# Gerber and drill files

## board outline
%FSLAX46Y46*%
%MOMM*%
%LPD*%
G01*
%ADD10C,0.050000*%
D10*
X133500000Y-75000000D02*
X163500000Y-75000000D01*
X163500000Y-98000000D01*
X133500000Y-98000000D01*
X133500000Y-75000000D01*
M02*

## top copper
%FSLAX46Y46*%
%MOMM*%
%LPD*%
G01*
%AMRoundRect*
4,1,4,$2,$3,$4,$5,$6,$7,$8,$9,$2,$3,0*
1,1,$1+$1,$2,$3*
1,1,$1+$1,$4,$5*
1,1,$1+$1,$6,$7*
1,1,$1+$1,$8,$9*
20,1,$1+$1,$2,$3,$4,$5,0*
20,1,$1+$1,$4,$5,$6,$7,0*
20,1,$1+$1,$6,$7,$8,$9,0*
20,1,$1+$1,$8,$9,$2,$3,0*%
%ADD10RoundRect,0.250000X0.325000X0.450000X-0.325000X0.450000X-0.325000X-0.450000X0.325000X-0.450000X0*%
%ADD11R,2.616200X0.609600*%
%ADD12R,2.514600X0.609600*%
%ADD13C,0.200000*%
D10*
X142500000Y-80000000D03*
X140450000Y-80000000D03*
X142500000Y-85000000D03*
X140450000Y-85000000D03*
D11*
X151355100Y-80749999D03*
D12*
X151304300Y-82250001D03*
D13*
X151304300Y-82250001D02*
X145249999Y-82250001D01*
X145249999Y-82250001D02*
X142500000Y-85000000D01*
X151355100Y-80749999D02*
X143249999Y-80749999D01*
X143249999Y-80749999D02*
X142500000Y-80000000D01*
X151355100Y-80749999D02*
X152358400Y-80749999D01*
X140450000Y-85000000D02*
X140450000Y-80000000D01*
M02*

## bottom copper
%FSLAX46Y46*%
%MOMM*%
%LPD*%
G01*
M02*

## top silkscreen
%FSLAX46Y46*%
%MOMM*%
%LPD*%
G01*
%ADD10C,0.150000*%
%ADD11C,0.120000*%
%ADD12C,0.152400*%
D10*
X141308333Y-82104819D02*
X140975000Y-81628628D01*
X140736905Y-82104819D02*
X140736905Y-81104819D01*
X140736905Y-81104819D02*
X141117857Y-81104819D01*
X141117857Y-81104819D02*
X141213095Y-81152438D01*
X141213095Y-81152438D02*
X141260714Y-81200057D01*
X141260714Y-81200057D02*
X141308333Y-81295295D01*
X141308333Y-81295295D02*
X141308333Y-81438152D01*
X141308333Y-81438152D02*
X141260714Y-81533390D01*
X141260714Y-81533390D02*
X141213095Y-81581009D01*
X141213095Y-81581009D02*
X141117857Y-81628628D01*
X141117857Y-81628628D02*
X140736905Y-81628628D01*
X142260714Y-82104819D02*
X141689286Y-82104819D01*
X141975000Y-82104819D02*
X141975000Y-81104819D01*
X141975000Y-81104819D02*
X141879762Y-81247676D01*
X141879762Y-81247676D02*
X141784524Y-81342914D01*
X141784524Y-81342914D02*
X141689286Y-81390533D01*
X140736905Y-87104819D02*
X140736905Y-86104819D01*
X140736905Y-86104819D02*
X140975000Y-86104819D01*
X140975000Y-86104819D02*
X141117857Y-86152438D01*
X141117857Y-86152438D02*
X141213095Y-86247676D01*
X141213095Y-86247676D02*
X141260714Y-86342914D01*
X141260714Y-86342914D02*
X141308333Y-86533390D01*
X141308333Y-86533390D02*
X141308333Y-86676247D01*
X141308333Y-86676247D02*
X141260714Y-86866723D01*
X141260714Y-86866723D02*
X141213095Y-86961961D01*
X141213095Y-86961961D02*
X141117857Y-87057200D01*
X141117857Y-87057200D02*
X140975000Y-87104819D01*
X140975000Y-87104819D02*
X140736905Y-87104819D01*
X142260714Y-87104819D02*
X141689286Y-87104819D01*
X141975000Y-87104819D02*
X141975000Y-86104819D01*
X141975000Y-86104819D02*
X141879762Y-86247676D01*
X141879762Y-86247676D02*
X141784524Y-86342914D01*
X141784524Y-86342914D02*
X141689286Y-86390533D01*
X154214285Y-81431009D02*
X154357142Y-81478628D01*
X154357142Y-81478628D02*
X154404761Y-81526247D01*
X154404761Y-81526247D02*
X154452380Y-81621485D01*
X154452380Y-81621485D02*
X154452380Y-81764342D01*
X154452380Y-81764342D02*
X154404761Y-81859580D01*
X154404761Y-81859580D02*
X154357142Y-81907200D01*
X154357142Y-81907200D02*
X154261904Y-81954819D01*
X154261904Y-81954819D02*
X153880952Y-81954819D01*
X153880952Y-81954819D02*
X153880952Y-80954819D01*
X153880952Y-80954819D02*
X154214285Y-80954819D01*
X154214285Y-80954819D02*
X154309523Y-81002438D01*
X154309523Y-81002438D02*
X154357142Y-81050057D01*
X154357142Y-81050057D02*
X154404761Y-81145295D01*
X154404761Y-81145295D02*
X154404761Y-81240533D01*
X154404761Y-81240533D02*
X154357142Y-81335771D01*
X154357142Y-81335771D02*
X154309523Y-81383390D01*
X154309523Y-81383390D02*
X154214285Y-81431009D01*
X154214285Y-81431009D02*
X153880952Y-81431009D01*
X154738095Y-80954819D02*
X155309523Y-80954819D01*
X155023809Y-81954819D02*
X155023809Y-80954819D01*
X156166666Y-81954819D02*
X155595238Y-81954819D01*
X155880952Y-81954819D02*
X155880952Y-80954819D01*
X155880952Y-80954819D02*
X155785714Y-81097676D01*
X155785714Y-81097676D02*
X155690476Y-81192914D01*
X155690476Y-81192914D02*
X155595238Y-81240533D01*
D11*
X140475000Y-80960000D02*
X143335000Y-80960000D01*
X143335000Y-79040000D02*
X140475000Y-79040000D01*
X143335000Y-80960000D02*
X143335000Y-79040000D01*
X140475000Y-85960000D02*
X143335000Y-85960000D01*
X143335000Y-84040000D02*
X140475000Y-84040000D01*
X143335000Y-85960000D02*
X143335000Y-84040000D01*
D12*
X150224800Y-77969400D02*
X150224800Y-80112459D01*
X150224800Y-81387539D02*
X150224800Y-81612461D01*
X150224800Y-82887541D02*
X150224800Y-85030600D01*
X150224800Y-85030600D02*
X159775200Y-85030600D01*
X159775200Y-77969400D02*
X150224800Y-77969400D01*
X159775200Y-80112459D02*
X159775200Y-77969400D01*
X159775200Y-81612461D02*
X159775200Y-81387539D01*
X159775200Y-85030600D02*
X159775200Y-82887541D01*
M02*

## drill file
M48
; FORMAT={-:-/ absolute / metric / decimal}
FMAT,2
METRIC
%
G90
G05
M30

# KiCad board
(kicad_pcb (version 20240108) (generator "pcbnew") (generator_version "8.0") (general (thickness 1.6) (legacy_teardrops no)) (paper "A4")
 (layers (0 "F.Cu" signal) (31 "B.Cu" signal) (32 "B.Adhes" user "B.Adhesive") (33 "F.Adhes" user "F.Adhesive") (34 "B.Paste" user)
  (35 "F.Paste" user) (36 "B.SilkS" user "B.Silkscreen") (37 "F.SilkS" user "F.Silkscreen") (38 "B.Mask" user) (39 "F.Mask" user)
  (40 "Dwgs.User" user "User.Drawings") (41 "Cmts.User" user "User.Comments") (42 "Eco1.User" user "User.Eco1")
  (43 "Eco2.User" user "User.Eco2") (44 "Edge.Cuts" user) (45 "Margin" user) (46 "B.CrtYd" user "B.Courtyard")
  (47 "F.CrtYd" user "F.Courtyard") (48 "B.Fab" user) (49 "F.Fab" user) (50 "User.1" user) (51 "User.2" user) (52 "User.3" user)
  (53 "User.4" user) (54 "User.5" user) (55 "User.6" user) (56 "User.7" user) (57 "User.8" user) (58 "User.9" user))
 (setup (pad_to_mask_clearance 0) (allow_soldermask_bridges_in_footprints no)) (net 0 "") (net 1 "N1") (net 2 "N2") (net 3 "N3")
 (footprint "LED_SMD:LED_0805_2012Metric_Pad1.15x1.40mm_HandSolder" (layer "F.Cu") (at 141.475 80 180)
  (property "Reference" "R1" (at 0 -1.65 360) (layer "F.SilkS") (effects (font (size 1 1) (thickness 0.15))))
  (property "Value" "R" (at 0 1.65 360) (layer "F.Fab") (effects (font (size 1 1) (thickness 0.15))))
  (fp_line (start 1 -0.96) (end -1.86 -0.96) (stroke (width 0.12) (type solid)) (layer "F.SilkS"))
  (fp_line (start -1.86 0.96) (end 1 0.96) (stroke (width 0.12) (type solid)) (layer "F.SilkS"))
  (fp_line (start -1.86 -0.96) (end -1.86 0.96) (stroke (width 0.12) (type solid)) (layer "F.SilkS"))
  (pad "1" smd roundrect (at -1.025 0 180) (size 1.15 1.4) (layers "F.Cu" "F.Paste" "F.Mask") (roundrect_rratio 0.217391) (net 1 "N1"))
  (pad "2" smd roundrect (at 1.025 0 180) (size 1.15 1.4) (layers "F.Cu" "F.Paste" "F.Mask") (roundrect_rratio 0.217391) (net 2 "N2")))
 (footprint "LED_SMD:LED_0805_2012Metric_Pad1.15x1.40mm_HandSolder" (layer "F.Cu") (at 141.475 85 180)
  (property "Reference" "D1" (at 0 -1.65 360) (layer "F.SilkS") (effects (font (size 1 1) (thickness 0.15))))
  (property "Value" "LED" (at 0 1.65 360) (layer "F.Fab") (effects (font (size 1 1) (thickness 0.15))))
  (fp_line (start 1 -0.96) (end -1.86 -0.96) (stroke (width 0.12) (type solid)) (layer "F.SilkS"))
  (fp_line (start -1.86 0.96) (end 1 0.96) (stroke (width 0.12) (type solid)) (layer "F.SilkS"))
  (fp_line (start -1.86 -0.96) (end -1.86 0.96) (stroke (width 0.12) (type solid)) (layer "F.SilkS"))
  (pad "1" smd roundrect (at -1.025 0 180) (size 1.15 1.4) (layers "F.Cu" "F.Paste" "F.Mask") (roundrect_rratio 0.217391) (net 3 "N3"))
  (pad "2" smd roundrect (at 1.025 0 180) (size 1.15 1.4) (layers "F.Cu" "F.Paste" "F.Mask") (roundrect_rratio 0.217391) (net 2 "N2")))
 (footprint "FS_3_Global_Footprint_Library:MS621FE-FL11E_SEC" (layer "F.Cu") (at 155 81.5)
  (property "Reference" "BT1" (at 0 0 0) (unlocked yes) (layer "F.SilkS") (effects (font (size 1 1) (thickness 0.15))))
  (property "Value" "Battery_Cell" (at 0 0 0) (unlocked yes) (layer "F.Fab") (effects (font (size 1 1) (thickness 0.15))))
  (fp_line (start -4.7752 -3.5306) (end -4.7752 -1.387541) (stroke (width 0.1524) (type solid)) (layer "F.SilkS"))
  (fp_line (start -4.7752 -0.112461) (end -4.7752 0.112461) (stroke (width 0.1524) (type solid)) (layer "F.SilkS"))
  (fp_line (start -4.7752 1.387541) (end -4.7752 3.5306) (stroke (width 0.1524) (type solid)) (layer "F.SilkS"))
  (fp_line (start -4.7752 3.5306) (end 4.7752 3.5306) (stroke (width 0.1524) (type solid)) (layer "F.SilkS"))
  (fp_line (start 4.7752 -3.5306) (end -4.7752 -3.5306) (stroke (width 0.1524) (type solid)) (layer "F.SilkS"))
  (fp_line (start 4.7752 -1.387541) (end 4.7752 -3.5306) (stroke (width 0.1524) (type solid)) (layer "F.SilkS"))
  (fp_line (start 4.7752 0.112461) (end 4.7752 -0.112461) (stroke (width 0.1524) (type solid)) (layer "F.SilkS"))
  (fp_line (start 4.7752 3.5306) (end 4.7752 1.387541) (stroke (width 0.1524) (type solid)) (layer "F.SilkS"))
  (pad "1" smd rect (at -3.6449 -0.750001) (size 2.6162 0.6096) (layers "F.Cu" "F.Paste" "F.Mask") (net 1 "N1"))
  (pad "2" smd rect (at -3.6957 0.750001) (size 2.5146 0.6096) (layers "F.Cu" "F.Paste" "F.Mask") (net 3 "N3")))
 (gr_rect (start 133.5 75) (end 163.5 98) (stroke (width 0.05) (type default)) (fill none) (layer "Edge.Cuts"))
 (segment (start 151.3043 82.250001) (end 145.249999 82.250001) (width 0.2) (layer "F.Cu") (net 3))
 (segment (start 145.249999 82.250001) (end 142.5 85) (width 0.2) (layer "F.Cu") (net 3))
 (segment (start 151.3551 80.749999) (end 143.249999 80.749999) (width 0.2) (layer "F.Cu") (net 1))
 (segment (start 143.249999 80.749999) (end 142.5 80) (width 0.2) (layer "F.Cu") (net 1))
 (segment (start 151.3551 80.749999) (end 152.3584 80.749999) (width 0.2) (layer "F.Cu") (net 1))
 (segment (start 140.45 85) (end 140.45 80) (width 0.2) (layer "F.Cu") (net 2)))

